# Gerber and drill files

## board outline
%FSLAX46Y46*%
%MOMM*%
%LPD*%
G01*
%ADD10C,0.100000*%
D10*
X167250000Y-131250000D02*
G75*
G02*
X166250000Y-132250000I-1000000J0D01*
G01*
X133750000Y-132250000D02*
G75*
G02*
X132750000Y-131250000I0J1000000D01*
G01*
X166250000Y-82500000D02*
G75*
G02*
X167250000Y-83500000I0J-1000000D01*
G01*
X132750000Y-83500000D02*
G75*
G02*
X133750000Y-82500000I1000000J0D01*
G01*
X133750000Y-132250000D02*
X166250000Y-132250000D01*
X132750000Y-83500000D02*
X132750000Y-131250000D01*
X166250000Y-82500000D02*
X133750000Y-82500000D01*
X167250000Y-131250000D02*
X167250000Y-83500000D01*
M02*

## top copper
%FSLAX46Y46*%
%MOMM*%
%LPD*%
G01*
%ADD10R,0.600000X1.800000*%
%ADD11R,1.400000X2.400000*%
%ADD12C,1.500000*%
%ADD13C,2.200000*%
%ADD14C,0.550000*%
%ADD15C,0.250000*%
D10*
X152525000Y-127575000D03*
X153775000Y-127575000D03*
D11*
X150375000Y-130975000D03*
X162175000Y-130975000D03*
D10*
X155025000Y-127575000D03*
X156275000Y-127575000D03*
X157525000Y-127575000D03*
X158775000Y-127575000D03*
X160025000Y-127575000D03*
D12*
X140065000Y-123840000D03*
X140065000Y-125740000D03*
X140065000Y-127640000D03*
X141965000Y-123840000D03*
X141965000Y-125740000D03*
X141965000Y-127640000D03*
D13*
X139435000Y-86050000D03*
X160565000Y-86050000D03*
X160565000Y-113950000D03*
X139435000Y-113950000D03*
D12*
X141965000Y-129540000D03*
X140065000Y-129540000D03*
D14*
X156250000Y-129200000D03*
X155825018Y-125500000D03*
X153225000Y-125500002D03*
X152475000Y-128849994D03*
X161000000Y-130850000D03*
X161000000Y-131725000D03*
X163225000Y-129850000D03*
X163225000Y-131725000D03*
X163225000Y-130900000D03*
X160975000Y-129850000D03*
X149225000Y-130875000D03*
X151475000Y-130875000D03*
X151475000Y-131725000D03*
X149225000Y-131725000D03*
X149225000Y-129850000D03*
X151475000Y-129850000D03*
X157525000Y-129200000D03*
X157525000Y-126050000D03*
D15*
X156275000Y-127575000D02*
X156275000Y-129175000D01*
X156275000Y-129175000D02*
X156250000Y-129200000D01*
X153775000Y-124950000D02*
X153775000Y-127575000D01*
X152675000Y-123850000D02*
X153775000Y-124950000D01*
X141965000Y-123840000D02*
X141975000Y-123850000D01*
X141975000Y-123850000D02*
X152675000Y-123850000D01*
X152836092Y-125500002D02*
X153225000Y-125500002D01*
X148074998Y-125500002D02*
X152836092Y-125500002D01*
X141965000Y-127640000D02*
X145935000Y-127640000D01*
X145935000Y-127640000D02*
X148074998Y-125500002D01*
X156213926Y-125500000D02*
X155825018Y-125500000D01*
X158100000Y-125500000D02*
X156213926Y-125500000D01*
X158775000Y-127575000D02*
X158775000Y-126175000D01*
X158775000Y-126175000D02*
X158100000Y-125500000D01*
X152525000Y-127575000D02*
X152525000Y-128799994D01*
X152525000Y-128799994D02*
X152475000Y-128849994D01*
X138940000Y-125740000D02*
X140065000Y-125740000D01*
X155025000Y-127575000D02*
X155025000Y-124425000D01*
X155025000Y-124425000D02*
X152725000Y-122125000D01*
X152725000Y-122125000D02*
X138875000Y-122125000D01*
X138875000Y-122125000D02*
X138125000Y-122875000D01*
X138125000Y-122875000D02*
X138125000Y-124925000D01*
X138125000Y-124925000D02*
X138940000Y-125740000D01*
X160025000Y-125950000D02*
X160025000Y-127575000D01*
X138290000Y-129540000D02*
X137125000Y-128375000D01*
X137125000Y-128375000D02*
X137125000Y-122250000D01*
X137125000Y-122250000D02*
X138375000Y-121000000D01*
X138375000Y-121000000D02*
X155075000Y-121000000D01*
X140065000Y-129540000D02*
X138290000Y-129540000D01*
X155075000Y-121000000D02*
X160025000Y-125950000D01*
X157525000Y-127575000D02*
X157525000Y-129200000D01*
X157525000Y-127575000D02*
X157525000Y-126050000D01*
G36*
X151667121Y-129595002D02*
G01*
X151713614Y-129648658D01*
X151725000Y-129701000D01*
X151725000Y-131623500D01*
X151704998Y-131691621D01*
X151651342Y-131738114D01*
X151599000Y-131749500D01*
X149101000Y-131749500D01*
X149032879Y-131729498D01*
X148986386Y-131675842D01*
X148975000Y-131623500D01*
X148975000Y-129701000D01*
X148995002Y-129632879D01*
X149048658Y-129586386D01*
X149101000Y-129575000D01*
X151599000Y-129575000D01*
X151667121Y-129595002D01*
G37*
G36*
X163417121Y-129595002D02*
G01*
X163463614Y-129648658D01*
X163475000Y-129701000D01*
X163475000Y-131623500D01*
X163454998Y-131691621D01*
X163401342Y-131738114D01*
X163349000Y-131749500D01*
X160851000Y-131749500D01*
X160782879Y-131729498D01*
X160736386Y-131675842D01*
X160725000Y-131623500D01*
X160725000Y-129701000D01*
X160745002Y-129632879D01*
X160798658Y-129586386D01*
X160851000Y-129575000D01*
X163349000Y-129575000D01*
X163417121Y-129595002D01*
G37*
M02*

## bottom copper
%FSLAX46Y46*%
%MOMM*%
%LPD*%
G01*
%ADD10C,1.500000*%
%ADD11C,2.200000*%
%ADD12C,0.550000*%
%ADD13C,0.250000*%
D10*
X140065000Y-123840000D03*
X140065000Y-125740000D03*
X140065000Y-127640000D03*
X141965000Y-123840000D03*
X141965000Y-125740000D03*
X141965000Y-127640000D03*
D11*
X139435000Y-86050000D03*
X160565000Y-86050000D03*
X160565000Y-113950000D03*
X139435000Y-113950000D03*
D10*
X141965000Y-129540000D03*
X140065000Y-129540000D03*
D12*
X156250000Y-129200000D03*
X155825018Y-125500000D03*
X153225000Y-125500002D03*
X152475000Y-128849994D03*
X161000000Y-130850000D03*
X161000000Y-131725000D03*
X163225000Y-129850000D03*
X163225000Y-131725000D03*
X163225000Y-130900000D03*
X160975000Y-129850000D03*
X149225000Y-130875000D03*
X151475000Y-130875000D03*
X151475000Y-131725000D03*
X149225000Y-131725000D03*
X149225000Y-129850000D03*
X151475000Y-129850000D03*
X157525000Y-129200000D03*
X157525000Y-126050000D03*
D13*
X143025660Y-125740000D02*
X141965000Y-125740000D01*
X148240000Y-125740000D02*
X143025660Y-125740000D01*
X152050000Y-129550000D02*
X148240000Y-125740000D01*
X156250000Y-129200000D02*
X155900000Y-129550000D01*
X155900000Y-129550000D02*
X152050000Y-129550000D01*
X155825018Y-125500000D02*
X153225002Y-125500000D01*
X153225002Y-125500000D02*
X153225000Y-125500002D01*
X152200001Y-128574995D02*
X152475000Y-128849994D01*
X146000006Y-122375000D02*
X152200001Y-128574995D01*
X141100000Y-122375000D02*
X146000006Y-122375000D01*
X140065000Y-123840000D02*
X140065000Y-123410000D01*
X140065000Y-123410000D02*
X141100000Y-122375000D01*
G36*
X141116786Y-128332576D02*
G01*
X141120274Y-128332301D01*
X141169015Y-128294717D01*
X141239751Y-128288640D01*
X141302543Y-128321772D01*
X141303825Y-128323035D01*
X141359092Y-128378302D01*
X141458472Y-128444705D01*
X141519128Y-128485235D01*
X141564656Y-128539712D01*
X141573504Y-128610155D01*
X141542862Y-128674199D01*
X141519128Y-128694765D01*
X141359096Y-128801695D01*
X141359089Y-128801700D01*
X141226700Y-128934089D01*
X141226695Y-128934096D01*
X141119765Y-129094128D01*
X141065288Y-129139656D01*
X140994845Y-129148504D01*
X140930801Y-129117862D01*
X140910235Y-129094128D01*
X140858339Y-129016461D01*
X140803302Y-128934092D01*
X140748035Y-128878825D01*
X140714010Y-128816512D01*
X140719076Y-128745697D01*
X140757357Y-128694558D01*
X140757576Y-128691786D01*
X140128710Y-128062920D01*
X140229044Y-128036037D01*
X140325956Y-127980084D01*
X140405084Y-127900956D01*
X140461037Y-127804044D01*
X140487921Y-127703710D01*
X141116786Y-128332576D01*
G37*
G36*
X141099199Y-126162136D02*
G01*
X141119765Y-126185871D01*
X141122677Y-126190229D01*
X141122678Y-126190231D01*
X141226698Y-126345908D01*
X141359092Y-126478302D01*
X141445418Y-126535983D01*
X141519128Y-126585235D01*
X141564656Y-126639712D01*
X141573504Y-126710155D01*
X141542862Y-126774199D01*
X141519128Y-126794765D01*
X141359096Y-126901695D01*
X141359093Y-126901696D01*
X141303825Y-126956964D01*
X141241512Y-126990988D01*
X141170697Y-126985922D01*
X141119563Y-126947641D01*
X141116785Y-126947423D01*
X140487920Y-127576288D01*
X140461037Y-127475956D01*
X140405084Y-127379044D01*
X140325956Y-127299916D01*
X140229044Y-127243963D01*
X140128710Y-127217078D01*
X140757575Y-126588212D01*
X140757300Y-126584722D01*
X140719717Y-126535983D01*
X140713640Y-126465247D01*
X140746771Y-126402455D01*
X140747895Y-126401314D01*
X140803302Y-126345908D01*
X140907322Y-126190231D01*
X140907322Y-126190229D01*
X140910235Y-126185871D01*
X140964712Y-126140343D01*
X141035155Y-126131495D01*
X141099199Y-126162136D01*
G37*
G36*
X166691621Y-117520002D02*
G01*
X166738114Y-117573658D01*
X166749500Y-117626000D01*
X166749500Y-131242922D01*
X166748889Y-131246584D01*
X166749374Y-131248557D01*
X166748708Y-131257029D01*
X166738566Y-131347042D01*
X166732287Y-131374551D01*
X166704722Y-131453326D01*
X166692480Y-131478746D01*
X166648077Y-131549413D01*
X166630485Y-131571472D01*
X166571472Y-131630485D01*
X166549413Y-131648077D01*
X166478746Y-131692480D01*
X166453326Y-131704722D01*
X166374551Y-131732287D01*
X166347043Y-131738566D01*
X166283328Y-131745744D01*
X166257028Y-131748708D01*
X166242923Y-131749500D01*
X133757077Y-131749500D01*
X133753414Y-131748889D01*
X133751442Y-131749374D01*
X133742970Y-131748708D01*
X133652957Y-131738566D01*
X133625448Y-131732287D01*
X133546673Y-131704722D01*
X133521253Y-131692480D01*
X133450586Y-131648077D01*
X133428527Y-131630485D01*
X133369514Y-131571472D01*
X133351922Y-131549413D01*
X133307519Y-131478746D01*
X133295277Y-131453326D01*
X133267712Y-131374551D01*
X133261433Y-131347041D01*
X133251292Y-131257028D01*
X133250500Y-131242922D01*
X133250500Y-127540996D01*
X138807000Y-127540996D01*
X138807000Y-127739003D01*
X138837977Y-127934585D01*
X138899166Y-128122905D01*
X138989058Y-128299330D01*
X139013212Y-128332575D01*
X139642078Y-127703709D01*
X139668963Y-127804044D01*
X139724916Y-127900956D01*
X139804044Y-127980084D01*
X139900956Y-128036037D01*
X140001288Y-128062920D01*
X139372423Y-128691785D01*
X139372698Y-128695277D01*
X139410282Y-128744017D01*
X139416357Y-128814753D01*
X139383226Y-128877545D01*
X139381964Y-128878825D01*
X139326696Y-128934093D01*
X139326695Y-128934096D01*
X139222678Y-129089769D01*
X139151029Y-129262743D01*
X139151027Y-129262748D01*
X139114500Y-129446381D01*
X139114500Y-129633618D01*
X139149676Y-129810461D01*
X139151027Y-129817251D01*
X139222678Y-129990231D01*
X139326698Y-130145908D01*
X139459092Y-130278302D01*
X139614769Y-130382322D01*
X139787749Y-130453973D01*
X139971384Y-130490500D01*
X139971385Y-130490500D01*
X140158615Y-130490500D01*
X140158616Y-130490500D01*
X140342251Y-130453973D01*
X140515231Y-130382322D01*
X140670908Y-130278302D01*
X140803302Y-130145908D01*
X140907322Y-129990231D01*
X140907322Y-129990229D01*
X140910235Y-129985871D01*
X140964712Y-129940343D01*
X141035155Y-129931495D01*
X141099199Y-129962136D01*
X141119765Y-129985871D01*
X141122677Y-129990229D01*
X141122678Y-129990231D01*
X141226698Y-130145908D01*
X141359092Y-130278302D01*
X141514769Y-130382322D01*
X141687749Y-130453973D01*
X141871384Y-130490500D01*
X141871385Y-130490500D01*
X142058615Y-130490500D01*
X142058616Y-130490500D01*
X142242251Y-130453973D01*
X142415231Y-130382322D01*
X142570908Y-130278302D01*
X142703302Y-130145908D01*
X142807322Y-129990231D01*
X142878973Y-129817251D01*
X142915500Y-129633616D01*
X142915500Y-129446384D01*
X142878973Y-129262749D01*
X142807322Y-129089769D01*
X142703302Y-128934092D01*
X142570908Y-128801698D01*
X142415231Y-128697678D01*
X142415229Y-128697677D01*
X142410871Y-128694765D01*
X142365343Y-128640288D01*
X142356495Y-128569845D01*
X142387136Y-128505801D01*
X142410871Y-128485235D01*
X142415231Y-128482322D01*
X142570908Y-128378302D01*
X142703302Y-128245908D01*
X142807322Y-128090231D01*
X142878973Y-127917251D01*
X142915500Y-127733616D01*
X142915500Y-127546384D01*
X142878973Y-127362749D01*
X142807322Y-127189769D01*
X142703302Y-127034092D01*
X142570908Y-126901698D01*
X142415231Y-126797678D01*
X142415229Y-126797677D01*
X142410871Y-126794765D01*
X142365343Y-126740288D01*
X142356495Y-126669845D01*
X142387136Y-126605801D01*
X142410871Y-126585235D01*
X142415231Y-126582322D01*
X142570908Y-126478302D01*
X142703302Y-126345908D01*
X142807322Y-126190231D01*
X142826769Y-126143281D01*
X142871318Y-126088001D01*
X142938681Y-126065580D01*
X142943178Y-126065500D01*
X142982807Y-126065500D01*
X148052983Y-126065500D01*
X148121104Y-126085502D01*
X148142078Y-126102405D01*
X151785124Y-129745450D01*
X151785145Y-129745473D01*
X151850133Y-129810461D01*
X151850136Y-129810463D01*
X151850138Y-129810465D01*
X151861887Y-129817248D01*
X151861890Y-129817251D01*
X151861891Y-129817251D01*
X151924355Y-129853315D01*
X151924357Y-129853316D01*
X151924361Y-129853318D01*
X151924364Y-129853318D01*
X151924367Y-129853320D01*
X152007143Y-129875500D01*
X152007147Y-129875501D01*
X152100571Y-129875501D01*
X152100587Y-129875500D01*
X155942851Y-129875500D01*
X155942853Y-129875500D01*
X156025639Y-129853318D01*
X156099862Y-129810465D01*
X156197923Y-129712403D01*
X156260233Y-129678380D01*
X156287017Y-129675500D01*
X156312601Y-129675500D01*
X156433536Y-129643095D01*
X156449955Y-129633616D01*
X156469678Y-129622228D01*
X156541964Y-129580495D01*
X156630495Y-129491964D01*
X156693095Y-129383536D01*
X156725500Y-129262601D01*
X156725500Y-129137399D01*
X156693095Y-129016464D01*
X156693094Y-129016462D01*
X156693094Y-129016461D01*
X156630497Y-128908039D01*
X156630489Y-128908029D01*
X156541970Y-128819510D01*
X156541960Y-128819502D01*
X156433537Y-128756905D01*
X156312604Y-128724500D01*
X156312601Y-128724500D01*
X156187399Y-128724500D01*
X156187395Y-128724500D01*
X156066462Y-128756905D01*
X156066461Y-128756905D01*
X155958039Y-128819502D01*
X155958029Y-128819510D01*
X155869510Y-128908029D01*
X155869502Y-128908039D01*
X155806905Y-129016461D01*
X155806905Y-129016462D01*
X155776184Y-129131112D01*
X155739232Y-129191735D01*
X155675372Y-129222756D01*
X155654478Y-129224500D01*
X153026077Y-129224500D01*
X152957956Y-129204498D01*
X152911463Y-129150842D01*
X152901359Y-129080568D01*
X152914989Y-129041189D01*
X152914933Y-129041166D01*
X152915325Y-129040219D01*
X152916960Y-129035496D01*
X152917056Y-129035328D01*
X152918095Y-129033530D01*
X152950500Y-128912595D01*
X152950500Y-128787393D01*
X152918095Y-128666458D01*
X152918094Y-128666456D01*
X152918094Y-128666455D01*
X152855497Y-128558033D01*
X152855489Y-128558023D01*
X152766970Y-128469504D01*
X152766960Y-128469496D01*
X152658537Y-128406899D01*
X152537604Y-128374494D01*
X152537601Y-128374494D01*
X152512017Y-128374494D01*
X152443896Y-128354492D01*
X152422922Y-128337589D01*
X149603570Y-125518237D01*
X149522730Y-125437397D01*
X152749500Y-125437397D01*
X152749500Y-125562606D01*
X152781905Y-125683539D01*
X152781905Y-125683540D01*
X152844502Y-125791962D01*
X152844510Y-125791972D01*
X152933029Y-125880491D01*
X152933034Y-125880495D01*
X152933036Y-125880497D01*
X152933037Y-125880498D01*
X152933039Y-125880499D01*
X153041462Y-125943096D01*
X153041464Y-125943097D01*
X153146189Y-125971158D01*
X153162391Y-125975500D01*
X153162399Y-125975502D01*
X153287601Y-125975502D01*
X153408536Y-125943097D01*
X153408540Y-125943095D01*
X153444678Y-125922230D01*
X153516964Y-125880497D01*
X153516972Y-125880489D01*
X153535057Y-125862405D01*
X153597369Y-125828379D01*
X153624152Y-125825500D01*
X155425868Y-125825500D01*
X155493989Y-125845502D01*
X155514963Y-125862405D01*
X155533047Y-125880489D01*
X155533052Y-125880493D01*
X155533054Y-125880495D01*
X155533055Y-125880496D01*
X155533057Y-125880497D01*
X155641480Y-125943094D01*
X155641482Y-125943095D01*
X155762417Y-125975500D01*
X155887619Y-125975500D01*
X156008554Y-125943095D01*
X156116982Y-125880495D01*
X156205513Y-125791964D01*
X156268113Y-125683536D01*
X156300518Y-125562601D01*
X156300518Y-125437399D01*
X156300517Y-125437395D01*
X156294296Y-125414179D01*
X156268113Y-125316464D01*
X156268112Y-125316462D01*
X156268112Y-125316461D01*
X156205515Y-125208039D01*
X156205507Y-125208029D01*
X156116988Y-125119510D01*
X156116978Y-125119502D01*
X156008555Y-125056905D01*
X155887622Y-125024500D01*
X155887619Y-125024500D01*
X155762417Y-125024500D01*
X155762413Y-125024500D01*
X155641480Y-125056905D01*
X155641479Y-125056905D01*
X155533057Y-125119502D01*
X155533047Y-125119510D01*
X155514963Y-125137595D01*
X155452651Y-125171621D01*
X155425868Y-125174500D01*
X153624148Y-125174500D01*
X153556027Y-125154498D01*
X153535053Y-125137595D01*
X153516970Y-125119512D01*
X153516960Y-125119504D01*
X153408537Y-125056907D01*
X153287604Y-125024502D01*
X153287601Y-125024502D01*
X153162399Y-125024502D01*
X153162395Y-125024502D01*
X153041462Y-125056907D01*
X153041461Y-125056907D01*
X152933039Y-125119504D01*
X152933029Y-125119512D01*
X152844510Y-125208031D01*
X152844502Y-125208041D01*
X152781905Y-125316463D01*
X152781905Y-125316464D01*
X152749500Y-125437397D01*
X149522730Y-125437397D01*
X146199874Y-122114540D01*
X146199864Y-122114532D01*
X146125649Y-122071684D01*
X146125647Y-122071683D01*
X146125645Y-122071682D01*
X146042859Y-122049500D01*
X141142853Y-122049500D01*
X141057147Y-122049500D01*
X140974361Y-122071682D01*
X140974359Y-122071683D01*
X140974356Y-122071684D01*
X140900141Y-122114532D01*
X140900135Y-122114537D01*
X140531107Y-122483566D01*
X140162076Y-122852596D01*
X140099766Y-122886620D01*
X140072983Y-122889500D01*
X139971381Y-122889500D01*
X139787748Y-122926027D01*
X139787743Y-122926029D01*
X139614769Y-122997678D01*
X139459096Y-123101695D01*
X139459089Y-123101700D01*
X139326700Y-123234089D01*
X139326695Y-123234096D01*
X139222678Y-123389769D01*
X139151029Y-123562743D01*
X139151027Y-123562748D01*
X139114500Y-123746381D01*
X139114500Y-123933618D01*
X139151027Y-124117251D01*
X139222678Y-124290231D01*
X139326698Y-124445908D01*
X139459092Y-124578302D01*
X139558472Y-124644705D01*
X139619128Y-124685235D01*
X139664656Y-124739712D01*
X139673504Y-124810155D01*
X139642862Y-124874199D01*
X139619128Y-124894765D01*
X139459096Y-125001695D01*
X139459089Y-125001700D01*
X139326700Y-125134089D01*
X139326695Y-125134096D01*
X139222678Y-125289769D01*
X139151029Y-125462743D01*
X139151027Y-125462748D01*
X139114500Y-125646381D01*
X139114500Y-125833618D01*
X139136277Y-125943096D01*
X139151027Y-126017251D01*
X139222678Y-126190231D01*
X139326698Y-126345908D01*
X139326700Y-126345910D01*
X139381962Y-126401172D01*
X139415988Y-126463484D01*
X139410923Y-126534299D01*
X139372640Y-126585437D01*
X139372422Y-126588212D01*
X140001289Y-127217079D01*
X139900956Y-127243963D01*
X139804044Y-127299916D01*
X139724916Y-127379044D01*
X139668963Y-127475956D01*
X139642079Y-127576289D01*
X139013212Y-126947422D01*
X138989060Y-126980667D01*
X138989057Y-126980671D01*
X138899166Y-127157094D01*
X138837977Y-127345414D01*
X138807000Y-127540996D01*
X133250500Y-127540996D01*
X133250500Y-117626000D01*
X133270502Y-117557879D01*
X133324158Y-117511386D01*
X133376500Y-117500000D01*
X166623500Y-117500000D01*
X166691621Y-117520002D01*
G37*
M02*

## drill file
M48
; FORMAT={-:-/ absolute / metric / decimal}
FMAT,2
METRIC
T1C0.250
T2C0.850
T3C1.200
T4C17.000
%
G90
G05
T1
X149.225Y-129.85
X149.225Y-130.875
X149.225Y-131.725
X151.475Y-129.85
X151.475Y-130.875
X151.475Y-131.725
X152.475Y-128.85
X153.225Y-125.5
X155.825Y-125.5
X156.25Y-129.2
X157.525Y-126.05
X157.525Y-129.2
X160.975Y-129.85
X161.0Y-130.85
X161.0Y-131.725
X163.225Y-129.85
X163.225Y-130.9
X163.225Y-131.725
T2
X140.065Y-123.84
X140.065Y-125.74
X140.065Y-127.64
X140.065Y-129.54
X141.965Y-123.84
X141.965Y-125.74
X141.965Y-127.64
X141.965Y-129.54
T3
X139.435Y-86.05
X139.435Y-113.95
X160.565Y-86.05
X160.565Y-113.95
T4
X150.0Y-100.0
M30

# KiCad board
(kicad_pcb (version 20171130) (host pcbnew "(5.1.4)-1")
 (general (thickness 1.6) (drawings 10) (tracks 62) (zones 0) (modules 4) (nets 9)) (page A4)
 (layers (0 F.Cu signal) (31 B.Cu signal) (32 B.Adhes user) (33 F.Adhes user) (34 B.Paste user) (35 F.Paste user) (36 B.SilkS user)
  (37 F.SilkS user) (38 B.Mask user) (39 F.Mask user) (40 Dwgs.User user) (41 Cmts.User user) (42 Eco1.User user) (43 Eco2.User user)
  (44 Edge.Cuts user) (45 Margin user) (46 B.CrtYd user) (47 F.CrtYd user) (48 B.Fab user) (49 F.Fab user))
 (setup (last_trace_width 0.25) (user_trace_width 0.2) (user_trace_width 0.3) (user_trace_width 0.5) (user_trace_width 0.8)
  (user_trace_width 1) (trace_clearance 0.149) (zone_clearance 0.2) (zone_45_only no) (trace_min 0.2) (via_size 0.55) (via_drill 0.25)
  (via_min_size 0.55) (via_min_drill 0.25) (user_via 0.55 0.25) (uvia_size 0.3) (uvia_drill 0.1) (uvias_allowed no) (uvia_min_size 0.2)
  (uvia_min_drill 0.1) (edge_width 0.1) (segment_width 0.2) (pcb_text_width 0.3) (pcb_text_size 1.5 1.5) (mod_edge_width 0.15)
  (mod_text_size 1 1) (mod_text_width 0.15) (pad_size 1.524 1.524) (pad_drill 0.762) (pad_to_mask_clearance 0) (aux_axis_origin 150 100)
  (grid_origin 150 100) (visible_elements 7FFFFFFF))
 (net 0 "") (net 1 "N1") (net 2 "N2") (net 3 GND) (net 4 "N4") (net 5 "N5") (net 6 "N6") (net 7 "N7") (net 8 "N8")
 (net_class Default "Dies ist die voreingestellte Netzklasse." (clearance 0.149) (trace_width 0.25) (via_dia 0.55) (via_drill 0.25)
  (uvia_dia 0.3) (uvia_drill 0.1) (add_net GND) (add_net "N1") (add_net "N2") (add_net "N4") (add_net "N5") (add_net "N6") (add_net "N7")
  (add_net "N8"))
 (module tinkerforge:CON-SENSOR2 (layer F.Cu) (at 156.275 132.175)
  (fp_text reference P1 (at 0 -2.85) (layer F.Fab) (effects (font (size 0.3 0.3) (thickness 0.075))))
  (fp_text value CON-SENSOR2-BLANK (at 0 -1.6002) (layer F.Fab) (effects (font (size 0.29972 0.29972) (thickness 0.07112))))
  (pad 1 smd rect (at -3.75 -4.6) (size 0.6 1.8) (layers F.Cu F.Paste F.Mask) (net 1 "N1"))
  (pad 2 smd rect (at -2.5 -4.6) (size 0.6 1.8) (layers F.Cu F.Paste F.Mask) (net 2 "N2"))
  (pad EP smd rect (at -5.9 -1.2) (size 1.4 2.4) (layers F.Cu F.Paste F.Mask) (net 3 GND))
  (pad EP smd rect (at 5.9 -1.2) (size 1.4 2.4) (layers F.Cu F.Paste F.Mask) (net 3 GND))
  (pad 3 smd rect (at -1.25 -4.6) (size 0.6 1.8) (layers F.Cu F.Paste F.Mask) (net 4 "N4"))
  (pad 4 smd rect (at 0 -4.6) (size 0.6 1.8) (layers F.Cu F.Paste F.Mask) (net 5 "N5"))
  (pad 5 smd rect (at 1.25 -4.6) (size 0.6 1.8) (layers F.Cu F.Paste F.Mask) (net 3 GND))
  (pad 6 smd rect (at 2.5 -4.6) (size 0.6 1.8) (layers F.Cu F.Paste F.Mask) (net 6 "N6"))
  (pad 7 smd rect (at 3.75 -4.6) (size 0.6 1.8) (layers F.Cu F.Paste F.Mask) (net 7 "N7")))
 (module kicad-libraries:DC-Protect (layer B.Cu) (at 150 100 180)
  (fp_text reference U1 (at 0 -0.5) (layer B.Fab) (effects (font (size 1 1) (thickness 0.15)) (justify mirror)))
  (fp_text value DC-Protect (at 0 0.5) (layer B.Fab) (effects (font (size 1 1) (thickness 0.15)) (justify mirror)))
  (pad 1 thru_hole circle (at 9.935 -23.84 180) (size 1.5 1.5) (drill 0.85) (layers *.Cu *.Mask) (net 1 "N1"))
  (pad 3 thru_hole circle (at 9.935 -25.74 180) (size 1.5 1.5) (drill 0.85) (layers *.Cu *.Mask) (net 4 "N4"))
  (pad 5 thru_hole circle (at 9.935 -27.64 180) (size 1.5 1.5) (drill 0.85) (layers *.Cu *.Mask) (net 3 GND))
  (pad 2 thru_hole circle (at 8.035 -23.84 180) (size 1.5 1.5) (drill 0.85) (layers *.Cu *.Mask) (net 2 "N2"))
  (pad 4 thru_hole circle (at 8.035 -25.74 180) (size 1.5 1.5) (drill 0.85) (layers *.Cu *.Mask) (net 5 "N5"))
  (pad 6 thru_hole circle (at 8.035 -27.64 180) (size 1.5 1.5) (drill 0.85) (layers *.Cu *.Mask) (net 6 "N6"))
  (pad "" np_thru_hole circle (at 0 0 180) (size 17 17) (drill 17) (layers *.Cu *.Mask))
  (pad "" thru_hole circle (at 10.565 13.95 180) (size 2.2 2.2) (drill 1.2) (layers *.Cu *.Mask))
  (pad "" thru_hole circle (at -10.565 13.95 180) (size 2.2 2.2) (drill 1.2) (layers *.Cu *.Mask))
  (pad "" thru_hole circle (at -10.565 -13.95 180) (size 2.2 2.2) (drill 1.2) (layers *.Cu *.Mask))
  (pad "" thru_hole circle (at 10.565 -13.95 180) (size 2.2 2.2) (drill 1.2) (layers *.Cu *.Mask))
  (pad 8 thru_hole circle (at 8.035 -29.54 180) (size 1.5 1.5) (drill 0.85) (layers *.Cu *.Mask) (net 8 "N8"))
  (pad 7 thru_hole circle (at 9.935 -29.54 180) (size 1.5 1.5) (drill 0.85) (layers *.Cu *.Mask) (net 7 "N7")))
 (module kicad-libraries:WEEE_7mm (layer F.Cu) (at 150 87.1 180)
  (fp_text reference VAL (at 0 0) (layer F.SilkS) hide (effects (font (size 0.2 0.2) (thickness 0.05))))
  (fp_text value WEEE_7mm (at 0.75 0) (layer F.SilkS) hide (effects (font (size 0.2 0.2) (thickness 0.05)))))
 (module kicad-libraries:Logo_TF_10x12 (layer F.Cu) (at 149.96 114.89 180)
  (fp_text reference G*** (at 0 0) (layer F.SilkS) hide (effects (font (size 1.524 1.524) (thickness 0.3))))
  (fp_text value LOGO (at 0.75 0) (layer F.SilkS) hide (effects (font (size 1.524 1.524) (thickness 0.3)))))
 (gr_arc (start 166.25 131.25) (end 166.25 132.25) (angle -90) (layer Edge.Cuts) (width 0.1))
 (gr_arc (start 133.75 131.25) (end 132.75 131.25) (angle -90) (layer Edge.Cuts) (width 0.1))
 (gr_arc (start 166.25 83.5) (end 167.25 83.5) (angle -90) (layer Edge.Cuts) (width 0.1))
 (gr_arc (start 133.75 83.5) (end 133.75 82.5) (angle -90) (layer Edge.Cuts) (width 0.1))
 (gr_line (start 133.75 132.25) (end 166.25 132.25) (layer Edge.Cuts) (width 0.1))
 (gr_line (start 132.75 83.5) (end 132.75 131.25) (layer Edge.Cuts) (width 0.1))
 (gr_line (start 166.25 82.5) (end 133.75 82.5) (layer Edge.Cuts) (width 0.1))
 (gr_line (start 167.25 131.25) (end 167.25 83.5) (layer Edge.Cuts) (width 0.1))
 (via (at 156.25 129.2) (size 0.55) (drill 0.25) (layers F.Cu B.Cu) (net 5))
 (segment (start 156.275 127.575) (end 156.275 129.175) (width 0.25) (layer F.Cu) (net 5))
 (segment (start 156.275 129.175) (end 156.25 129.2) (width 0.25) (layer F.Cu) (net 5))
 (segment (start 143.02566 125.74) (end 141.965 125.74) (width 0.25) (layer B.Cu) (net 5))
 (segment (start 148.24 125.74) (end 143.02566 125.74) (width 0.25) (layer B.Cu) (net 5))
 (segment (start 152.05 129.55) (end 148.24 125.74) (width 0.25) (layer B.Cu) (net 5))
 (segment (start 156.25 129.2) (end 155.9 129.55) (width 0.25) (layer B.Cu) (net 5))
 (segment (start 155.9 129.55) (end 152.05 129.55) (width 0.25) (layer B.Cu) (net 5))
 (segment (start 153.775 124.95) (end 153.775 127.575) (width 0.25) (layer F.Cu) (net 2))
 (segment (start 152.675 123.85) (end 153.775 124.95) (width 0.25) (layer F.Cu) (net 2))
 (segment (start 141.965 123.84) (end 141.975 123.85) (width 0.25) (layer F.Cu) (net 2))
 (segment (start 141.975 123.85) (end 152.675 123.85) (width 0.25) (layer F.Cu) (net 2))
 (via (at 155.825018 125.5) (size 0.55) (drill 0.25) (layers F.Cu B.Cu) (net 6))
 (via (at 153.225 125.500002) (size 0.55) (drill 0.25) (layers F.Cu B.Cu) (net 6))
 (segment (start 155.825018 125.5) (end 153.225002 125.5) (width 0.25) (layer B.Cu) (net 6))
 (segment (start 153.225002 125.5) (end 153.225 125.500002) (width 0.25) (layer B.Cu) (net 6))
 (segment (start 152.836092 125.500002) (end 153.225 125.500002) (width 0.25) (layer F.Cu) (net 6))
 (segment (start 148.074998 125.500002) (end 152.836092 125.500002) (width 0.25) (layer F.Cu) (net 6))
 (segment (start 141.965 127.64) (end 145.935 127.64) (width 0.25) (layer F.Cu) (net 6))
 (segment (start 145.935 127.64) (end 148.074998 125.500002) (width 0.25) (layer F.Cu) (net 6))
 (segment (start 156.213926 125.5) (end 155.825018 125.5) (width 0.25) (layer F.Cu) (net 6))
 (segment (start 158.1 125.5) (end 156.213926 125.5) (width 0.25) (layer F.Cu) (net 6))
 (segment (start 158.775 127.575) (end 158.775 126.175) (width 0.25) (layer F.Cu) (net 6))
 (segment (start 158.775 126.175) (end 158.1 125.5) (width 0.25) (layer F.Cu) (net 6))
 (segment (start 152.525 127.575) (end 152.525 128.799994) (width 0.25) (layer F.Cu) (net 1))
 (segment (start 152.525 128.799994) (end 152.475 128.849994) (width 0.25) (layer F.Cu) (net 1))
 (via (at 152.475 128.849994) (size 0.55) (drill 0.25) (layers F.Cu B.Cu) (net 1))
 (segment (start 152.200001 128.574995) (end 152.475 128.849994) (width 0.25) (layer B.Cu) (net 1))
 (segment (start 146.000006 122.375) (end 152.200001 128.574995) (width 0.25) (layer B.Cu) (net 1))
 (segment (start 141.1 122.375) (end 146.000006 122.375) (width 0.25) (layer B.Cu) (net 1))
 (segment (start 140.065 123.84) (end 140.065 123.41) (width 0.25) (layer B.Cu) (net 1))
 (segment (start 140.065 123.41) (end 141.1 122.375) (width 0.25) (layer B.Cu) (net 1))
 (segment (start 138.94 125.74) (end 140.065 125.74) (width 0.25) (layer F.Cu) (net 4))
 (segment (start 155.025 127.575) (end 155.025 124.425) (width 0.25) (layer F.Cu) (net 4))
 (segment (start 155.025 124.425) (end 152.725 122.125) (width 0.25) (layer F.Cu) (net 4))
 (segment (start 152.725 122.125) (end 138.875 122.125) (width 0.25) (layer F.Cu) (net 4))
 (segment (start 138.875 122.125) (end 138.125 122.875) (width 0.25) (layer F.Cu) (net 4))
 (segment (start 138.125 122.875) (end 138.125 124.925) (width 0.25) (layer F.Cu) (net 4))
 (segment (start 138.125 124.925) (end 138.94 125.74) (width 0.25) (layer F.Cu) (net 4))
 (segment (start 160.025 125.95) (end 160.025 127.575) (width 0.25) (layer F.Cu) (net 7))
 (segment (start 138.29 129.54) (end 137.125 128.375) (width 0.25) (layer F.Cu) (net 7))
 (segment (start 137.125 128.375) (end 137.125 122.25) (width 0.25) (layer F.Cu) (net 7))
 (segment (start 137.125 122.25) (end 138.375 121) (width 0.25) (layer F.Cu) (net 7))
 (segment (start 138.375 121) (end 155.075 121) (width 0.25) (layer F.Cu) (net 7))
 (segment (start 140.065 129.54) (end 138.29 129.54) (width 0.25) (layer F.Cu) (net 7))
 (segment (start 155.075 121) (end 160.025 125.95) (width 0.25) (layer F.Cu) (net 7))
 (via (at 161 130.85) (size 0.55) (drill 0.25) (layers F.Cu B.Cu) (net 3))
 (via (at 161 131.725) (size 0.55) (drill 0.25) (layers F.Cu B.Cu) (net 3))
 (via (at 163.225 129.85) (size 0.55) (drill 0.25) (layers F.Cu B.Cu) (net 3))
 (via (at 163.225 131.725) (size 0.55) (drill 0.25) (layers F.Cu B.Cu) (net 3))
 (via (at 163.225 130.9) (size 0.55) (drill 0.25) (layers F.Cu B.Cu) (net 3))
 (via (at 160.975 129.85) (size 0.55) (drill 0.25) (layers F.Cu B.Cu) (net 3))
 (via (at 149.225 130.875) (size 0.55) (drill 0.25) (layers F.Cu B.Cu) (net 3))
 (via (at 151.475 130.875) (size 0.55) (drill 0.25) (layers F.Cu B.Cu) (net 3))
 (via (at 151.475 131.725) (size 0.55) (drill 0.25) (layers F.Cu B.Cu) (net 3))
 (via (at 149.225 131.725) (size 0.55) (drill 0.25) (layers F.Cu B.Cu) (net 3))
 (via (at 149.225 129.85) (size 0.55) (drill 0.25) (layers F.Cu B.Cu) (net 3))
 (via (at 151.475 129.85) (size 0.55) (drill 0.25) (layers F.Cu B.Cu) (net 3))
 (via (at 157.525 129.2) (size 0.55) (drill 0.25) (layers F.Cu B.Cu) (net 3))
 (segment (start 157.525 127.575) (end 157.525 129.2) (width 0.25) (layer F.Cu) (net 3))
 (via (at 157.525 126.05) (size 0.55) (drill 0.25) (layers F.Cu B.Cu) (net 3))
 (segment (start 157.525 127.575) (end 157.525 126.05) (width 0.25) (layer F.Cu) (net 3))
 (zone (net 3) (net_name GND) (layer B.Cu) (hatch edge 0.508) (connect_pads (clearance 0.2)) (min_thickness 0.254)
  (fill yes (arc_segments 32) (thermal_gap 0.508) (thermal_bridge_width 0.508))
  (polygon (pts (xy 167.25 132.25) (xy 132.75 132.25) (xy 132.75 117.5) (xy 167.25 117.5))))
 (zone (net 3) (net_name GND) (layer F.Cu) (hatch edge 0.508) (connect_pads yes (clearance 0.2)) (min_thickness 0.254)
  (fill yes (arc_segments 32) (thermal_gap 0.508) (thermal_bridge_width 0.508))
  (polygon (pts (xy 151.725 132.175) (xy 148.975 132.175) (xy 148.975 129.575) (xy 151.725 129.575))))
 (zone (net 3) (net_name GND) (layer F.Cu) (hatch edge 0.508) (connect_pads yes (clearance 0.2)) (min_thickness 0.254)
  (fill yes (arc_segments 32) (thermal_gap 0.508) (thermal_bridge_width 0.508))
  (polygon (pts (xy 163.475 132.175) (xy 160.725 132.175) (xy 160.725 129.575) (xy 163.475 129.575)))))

